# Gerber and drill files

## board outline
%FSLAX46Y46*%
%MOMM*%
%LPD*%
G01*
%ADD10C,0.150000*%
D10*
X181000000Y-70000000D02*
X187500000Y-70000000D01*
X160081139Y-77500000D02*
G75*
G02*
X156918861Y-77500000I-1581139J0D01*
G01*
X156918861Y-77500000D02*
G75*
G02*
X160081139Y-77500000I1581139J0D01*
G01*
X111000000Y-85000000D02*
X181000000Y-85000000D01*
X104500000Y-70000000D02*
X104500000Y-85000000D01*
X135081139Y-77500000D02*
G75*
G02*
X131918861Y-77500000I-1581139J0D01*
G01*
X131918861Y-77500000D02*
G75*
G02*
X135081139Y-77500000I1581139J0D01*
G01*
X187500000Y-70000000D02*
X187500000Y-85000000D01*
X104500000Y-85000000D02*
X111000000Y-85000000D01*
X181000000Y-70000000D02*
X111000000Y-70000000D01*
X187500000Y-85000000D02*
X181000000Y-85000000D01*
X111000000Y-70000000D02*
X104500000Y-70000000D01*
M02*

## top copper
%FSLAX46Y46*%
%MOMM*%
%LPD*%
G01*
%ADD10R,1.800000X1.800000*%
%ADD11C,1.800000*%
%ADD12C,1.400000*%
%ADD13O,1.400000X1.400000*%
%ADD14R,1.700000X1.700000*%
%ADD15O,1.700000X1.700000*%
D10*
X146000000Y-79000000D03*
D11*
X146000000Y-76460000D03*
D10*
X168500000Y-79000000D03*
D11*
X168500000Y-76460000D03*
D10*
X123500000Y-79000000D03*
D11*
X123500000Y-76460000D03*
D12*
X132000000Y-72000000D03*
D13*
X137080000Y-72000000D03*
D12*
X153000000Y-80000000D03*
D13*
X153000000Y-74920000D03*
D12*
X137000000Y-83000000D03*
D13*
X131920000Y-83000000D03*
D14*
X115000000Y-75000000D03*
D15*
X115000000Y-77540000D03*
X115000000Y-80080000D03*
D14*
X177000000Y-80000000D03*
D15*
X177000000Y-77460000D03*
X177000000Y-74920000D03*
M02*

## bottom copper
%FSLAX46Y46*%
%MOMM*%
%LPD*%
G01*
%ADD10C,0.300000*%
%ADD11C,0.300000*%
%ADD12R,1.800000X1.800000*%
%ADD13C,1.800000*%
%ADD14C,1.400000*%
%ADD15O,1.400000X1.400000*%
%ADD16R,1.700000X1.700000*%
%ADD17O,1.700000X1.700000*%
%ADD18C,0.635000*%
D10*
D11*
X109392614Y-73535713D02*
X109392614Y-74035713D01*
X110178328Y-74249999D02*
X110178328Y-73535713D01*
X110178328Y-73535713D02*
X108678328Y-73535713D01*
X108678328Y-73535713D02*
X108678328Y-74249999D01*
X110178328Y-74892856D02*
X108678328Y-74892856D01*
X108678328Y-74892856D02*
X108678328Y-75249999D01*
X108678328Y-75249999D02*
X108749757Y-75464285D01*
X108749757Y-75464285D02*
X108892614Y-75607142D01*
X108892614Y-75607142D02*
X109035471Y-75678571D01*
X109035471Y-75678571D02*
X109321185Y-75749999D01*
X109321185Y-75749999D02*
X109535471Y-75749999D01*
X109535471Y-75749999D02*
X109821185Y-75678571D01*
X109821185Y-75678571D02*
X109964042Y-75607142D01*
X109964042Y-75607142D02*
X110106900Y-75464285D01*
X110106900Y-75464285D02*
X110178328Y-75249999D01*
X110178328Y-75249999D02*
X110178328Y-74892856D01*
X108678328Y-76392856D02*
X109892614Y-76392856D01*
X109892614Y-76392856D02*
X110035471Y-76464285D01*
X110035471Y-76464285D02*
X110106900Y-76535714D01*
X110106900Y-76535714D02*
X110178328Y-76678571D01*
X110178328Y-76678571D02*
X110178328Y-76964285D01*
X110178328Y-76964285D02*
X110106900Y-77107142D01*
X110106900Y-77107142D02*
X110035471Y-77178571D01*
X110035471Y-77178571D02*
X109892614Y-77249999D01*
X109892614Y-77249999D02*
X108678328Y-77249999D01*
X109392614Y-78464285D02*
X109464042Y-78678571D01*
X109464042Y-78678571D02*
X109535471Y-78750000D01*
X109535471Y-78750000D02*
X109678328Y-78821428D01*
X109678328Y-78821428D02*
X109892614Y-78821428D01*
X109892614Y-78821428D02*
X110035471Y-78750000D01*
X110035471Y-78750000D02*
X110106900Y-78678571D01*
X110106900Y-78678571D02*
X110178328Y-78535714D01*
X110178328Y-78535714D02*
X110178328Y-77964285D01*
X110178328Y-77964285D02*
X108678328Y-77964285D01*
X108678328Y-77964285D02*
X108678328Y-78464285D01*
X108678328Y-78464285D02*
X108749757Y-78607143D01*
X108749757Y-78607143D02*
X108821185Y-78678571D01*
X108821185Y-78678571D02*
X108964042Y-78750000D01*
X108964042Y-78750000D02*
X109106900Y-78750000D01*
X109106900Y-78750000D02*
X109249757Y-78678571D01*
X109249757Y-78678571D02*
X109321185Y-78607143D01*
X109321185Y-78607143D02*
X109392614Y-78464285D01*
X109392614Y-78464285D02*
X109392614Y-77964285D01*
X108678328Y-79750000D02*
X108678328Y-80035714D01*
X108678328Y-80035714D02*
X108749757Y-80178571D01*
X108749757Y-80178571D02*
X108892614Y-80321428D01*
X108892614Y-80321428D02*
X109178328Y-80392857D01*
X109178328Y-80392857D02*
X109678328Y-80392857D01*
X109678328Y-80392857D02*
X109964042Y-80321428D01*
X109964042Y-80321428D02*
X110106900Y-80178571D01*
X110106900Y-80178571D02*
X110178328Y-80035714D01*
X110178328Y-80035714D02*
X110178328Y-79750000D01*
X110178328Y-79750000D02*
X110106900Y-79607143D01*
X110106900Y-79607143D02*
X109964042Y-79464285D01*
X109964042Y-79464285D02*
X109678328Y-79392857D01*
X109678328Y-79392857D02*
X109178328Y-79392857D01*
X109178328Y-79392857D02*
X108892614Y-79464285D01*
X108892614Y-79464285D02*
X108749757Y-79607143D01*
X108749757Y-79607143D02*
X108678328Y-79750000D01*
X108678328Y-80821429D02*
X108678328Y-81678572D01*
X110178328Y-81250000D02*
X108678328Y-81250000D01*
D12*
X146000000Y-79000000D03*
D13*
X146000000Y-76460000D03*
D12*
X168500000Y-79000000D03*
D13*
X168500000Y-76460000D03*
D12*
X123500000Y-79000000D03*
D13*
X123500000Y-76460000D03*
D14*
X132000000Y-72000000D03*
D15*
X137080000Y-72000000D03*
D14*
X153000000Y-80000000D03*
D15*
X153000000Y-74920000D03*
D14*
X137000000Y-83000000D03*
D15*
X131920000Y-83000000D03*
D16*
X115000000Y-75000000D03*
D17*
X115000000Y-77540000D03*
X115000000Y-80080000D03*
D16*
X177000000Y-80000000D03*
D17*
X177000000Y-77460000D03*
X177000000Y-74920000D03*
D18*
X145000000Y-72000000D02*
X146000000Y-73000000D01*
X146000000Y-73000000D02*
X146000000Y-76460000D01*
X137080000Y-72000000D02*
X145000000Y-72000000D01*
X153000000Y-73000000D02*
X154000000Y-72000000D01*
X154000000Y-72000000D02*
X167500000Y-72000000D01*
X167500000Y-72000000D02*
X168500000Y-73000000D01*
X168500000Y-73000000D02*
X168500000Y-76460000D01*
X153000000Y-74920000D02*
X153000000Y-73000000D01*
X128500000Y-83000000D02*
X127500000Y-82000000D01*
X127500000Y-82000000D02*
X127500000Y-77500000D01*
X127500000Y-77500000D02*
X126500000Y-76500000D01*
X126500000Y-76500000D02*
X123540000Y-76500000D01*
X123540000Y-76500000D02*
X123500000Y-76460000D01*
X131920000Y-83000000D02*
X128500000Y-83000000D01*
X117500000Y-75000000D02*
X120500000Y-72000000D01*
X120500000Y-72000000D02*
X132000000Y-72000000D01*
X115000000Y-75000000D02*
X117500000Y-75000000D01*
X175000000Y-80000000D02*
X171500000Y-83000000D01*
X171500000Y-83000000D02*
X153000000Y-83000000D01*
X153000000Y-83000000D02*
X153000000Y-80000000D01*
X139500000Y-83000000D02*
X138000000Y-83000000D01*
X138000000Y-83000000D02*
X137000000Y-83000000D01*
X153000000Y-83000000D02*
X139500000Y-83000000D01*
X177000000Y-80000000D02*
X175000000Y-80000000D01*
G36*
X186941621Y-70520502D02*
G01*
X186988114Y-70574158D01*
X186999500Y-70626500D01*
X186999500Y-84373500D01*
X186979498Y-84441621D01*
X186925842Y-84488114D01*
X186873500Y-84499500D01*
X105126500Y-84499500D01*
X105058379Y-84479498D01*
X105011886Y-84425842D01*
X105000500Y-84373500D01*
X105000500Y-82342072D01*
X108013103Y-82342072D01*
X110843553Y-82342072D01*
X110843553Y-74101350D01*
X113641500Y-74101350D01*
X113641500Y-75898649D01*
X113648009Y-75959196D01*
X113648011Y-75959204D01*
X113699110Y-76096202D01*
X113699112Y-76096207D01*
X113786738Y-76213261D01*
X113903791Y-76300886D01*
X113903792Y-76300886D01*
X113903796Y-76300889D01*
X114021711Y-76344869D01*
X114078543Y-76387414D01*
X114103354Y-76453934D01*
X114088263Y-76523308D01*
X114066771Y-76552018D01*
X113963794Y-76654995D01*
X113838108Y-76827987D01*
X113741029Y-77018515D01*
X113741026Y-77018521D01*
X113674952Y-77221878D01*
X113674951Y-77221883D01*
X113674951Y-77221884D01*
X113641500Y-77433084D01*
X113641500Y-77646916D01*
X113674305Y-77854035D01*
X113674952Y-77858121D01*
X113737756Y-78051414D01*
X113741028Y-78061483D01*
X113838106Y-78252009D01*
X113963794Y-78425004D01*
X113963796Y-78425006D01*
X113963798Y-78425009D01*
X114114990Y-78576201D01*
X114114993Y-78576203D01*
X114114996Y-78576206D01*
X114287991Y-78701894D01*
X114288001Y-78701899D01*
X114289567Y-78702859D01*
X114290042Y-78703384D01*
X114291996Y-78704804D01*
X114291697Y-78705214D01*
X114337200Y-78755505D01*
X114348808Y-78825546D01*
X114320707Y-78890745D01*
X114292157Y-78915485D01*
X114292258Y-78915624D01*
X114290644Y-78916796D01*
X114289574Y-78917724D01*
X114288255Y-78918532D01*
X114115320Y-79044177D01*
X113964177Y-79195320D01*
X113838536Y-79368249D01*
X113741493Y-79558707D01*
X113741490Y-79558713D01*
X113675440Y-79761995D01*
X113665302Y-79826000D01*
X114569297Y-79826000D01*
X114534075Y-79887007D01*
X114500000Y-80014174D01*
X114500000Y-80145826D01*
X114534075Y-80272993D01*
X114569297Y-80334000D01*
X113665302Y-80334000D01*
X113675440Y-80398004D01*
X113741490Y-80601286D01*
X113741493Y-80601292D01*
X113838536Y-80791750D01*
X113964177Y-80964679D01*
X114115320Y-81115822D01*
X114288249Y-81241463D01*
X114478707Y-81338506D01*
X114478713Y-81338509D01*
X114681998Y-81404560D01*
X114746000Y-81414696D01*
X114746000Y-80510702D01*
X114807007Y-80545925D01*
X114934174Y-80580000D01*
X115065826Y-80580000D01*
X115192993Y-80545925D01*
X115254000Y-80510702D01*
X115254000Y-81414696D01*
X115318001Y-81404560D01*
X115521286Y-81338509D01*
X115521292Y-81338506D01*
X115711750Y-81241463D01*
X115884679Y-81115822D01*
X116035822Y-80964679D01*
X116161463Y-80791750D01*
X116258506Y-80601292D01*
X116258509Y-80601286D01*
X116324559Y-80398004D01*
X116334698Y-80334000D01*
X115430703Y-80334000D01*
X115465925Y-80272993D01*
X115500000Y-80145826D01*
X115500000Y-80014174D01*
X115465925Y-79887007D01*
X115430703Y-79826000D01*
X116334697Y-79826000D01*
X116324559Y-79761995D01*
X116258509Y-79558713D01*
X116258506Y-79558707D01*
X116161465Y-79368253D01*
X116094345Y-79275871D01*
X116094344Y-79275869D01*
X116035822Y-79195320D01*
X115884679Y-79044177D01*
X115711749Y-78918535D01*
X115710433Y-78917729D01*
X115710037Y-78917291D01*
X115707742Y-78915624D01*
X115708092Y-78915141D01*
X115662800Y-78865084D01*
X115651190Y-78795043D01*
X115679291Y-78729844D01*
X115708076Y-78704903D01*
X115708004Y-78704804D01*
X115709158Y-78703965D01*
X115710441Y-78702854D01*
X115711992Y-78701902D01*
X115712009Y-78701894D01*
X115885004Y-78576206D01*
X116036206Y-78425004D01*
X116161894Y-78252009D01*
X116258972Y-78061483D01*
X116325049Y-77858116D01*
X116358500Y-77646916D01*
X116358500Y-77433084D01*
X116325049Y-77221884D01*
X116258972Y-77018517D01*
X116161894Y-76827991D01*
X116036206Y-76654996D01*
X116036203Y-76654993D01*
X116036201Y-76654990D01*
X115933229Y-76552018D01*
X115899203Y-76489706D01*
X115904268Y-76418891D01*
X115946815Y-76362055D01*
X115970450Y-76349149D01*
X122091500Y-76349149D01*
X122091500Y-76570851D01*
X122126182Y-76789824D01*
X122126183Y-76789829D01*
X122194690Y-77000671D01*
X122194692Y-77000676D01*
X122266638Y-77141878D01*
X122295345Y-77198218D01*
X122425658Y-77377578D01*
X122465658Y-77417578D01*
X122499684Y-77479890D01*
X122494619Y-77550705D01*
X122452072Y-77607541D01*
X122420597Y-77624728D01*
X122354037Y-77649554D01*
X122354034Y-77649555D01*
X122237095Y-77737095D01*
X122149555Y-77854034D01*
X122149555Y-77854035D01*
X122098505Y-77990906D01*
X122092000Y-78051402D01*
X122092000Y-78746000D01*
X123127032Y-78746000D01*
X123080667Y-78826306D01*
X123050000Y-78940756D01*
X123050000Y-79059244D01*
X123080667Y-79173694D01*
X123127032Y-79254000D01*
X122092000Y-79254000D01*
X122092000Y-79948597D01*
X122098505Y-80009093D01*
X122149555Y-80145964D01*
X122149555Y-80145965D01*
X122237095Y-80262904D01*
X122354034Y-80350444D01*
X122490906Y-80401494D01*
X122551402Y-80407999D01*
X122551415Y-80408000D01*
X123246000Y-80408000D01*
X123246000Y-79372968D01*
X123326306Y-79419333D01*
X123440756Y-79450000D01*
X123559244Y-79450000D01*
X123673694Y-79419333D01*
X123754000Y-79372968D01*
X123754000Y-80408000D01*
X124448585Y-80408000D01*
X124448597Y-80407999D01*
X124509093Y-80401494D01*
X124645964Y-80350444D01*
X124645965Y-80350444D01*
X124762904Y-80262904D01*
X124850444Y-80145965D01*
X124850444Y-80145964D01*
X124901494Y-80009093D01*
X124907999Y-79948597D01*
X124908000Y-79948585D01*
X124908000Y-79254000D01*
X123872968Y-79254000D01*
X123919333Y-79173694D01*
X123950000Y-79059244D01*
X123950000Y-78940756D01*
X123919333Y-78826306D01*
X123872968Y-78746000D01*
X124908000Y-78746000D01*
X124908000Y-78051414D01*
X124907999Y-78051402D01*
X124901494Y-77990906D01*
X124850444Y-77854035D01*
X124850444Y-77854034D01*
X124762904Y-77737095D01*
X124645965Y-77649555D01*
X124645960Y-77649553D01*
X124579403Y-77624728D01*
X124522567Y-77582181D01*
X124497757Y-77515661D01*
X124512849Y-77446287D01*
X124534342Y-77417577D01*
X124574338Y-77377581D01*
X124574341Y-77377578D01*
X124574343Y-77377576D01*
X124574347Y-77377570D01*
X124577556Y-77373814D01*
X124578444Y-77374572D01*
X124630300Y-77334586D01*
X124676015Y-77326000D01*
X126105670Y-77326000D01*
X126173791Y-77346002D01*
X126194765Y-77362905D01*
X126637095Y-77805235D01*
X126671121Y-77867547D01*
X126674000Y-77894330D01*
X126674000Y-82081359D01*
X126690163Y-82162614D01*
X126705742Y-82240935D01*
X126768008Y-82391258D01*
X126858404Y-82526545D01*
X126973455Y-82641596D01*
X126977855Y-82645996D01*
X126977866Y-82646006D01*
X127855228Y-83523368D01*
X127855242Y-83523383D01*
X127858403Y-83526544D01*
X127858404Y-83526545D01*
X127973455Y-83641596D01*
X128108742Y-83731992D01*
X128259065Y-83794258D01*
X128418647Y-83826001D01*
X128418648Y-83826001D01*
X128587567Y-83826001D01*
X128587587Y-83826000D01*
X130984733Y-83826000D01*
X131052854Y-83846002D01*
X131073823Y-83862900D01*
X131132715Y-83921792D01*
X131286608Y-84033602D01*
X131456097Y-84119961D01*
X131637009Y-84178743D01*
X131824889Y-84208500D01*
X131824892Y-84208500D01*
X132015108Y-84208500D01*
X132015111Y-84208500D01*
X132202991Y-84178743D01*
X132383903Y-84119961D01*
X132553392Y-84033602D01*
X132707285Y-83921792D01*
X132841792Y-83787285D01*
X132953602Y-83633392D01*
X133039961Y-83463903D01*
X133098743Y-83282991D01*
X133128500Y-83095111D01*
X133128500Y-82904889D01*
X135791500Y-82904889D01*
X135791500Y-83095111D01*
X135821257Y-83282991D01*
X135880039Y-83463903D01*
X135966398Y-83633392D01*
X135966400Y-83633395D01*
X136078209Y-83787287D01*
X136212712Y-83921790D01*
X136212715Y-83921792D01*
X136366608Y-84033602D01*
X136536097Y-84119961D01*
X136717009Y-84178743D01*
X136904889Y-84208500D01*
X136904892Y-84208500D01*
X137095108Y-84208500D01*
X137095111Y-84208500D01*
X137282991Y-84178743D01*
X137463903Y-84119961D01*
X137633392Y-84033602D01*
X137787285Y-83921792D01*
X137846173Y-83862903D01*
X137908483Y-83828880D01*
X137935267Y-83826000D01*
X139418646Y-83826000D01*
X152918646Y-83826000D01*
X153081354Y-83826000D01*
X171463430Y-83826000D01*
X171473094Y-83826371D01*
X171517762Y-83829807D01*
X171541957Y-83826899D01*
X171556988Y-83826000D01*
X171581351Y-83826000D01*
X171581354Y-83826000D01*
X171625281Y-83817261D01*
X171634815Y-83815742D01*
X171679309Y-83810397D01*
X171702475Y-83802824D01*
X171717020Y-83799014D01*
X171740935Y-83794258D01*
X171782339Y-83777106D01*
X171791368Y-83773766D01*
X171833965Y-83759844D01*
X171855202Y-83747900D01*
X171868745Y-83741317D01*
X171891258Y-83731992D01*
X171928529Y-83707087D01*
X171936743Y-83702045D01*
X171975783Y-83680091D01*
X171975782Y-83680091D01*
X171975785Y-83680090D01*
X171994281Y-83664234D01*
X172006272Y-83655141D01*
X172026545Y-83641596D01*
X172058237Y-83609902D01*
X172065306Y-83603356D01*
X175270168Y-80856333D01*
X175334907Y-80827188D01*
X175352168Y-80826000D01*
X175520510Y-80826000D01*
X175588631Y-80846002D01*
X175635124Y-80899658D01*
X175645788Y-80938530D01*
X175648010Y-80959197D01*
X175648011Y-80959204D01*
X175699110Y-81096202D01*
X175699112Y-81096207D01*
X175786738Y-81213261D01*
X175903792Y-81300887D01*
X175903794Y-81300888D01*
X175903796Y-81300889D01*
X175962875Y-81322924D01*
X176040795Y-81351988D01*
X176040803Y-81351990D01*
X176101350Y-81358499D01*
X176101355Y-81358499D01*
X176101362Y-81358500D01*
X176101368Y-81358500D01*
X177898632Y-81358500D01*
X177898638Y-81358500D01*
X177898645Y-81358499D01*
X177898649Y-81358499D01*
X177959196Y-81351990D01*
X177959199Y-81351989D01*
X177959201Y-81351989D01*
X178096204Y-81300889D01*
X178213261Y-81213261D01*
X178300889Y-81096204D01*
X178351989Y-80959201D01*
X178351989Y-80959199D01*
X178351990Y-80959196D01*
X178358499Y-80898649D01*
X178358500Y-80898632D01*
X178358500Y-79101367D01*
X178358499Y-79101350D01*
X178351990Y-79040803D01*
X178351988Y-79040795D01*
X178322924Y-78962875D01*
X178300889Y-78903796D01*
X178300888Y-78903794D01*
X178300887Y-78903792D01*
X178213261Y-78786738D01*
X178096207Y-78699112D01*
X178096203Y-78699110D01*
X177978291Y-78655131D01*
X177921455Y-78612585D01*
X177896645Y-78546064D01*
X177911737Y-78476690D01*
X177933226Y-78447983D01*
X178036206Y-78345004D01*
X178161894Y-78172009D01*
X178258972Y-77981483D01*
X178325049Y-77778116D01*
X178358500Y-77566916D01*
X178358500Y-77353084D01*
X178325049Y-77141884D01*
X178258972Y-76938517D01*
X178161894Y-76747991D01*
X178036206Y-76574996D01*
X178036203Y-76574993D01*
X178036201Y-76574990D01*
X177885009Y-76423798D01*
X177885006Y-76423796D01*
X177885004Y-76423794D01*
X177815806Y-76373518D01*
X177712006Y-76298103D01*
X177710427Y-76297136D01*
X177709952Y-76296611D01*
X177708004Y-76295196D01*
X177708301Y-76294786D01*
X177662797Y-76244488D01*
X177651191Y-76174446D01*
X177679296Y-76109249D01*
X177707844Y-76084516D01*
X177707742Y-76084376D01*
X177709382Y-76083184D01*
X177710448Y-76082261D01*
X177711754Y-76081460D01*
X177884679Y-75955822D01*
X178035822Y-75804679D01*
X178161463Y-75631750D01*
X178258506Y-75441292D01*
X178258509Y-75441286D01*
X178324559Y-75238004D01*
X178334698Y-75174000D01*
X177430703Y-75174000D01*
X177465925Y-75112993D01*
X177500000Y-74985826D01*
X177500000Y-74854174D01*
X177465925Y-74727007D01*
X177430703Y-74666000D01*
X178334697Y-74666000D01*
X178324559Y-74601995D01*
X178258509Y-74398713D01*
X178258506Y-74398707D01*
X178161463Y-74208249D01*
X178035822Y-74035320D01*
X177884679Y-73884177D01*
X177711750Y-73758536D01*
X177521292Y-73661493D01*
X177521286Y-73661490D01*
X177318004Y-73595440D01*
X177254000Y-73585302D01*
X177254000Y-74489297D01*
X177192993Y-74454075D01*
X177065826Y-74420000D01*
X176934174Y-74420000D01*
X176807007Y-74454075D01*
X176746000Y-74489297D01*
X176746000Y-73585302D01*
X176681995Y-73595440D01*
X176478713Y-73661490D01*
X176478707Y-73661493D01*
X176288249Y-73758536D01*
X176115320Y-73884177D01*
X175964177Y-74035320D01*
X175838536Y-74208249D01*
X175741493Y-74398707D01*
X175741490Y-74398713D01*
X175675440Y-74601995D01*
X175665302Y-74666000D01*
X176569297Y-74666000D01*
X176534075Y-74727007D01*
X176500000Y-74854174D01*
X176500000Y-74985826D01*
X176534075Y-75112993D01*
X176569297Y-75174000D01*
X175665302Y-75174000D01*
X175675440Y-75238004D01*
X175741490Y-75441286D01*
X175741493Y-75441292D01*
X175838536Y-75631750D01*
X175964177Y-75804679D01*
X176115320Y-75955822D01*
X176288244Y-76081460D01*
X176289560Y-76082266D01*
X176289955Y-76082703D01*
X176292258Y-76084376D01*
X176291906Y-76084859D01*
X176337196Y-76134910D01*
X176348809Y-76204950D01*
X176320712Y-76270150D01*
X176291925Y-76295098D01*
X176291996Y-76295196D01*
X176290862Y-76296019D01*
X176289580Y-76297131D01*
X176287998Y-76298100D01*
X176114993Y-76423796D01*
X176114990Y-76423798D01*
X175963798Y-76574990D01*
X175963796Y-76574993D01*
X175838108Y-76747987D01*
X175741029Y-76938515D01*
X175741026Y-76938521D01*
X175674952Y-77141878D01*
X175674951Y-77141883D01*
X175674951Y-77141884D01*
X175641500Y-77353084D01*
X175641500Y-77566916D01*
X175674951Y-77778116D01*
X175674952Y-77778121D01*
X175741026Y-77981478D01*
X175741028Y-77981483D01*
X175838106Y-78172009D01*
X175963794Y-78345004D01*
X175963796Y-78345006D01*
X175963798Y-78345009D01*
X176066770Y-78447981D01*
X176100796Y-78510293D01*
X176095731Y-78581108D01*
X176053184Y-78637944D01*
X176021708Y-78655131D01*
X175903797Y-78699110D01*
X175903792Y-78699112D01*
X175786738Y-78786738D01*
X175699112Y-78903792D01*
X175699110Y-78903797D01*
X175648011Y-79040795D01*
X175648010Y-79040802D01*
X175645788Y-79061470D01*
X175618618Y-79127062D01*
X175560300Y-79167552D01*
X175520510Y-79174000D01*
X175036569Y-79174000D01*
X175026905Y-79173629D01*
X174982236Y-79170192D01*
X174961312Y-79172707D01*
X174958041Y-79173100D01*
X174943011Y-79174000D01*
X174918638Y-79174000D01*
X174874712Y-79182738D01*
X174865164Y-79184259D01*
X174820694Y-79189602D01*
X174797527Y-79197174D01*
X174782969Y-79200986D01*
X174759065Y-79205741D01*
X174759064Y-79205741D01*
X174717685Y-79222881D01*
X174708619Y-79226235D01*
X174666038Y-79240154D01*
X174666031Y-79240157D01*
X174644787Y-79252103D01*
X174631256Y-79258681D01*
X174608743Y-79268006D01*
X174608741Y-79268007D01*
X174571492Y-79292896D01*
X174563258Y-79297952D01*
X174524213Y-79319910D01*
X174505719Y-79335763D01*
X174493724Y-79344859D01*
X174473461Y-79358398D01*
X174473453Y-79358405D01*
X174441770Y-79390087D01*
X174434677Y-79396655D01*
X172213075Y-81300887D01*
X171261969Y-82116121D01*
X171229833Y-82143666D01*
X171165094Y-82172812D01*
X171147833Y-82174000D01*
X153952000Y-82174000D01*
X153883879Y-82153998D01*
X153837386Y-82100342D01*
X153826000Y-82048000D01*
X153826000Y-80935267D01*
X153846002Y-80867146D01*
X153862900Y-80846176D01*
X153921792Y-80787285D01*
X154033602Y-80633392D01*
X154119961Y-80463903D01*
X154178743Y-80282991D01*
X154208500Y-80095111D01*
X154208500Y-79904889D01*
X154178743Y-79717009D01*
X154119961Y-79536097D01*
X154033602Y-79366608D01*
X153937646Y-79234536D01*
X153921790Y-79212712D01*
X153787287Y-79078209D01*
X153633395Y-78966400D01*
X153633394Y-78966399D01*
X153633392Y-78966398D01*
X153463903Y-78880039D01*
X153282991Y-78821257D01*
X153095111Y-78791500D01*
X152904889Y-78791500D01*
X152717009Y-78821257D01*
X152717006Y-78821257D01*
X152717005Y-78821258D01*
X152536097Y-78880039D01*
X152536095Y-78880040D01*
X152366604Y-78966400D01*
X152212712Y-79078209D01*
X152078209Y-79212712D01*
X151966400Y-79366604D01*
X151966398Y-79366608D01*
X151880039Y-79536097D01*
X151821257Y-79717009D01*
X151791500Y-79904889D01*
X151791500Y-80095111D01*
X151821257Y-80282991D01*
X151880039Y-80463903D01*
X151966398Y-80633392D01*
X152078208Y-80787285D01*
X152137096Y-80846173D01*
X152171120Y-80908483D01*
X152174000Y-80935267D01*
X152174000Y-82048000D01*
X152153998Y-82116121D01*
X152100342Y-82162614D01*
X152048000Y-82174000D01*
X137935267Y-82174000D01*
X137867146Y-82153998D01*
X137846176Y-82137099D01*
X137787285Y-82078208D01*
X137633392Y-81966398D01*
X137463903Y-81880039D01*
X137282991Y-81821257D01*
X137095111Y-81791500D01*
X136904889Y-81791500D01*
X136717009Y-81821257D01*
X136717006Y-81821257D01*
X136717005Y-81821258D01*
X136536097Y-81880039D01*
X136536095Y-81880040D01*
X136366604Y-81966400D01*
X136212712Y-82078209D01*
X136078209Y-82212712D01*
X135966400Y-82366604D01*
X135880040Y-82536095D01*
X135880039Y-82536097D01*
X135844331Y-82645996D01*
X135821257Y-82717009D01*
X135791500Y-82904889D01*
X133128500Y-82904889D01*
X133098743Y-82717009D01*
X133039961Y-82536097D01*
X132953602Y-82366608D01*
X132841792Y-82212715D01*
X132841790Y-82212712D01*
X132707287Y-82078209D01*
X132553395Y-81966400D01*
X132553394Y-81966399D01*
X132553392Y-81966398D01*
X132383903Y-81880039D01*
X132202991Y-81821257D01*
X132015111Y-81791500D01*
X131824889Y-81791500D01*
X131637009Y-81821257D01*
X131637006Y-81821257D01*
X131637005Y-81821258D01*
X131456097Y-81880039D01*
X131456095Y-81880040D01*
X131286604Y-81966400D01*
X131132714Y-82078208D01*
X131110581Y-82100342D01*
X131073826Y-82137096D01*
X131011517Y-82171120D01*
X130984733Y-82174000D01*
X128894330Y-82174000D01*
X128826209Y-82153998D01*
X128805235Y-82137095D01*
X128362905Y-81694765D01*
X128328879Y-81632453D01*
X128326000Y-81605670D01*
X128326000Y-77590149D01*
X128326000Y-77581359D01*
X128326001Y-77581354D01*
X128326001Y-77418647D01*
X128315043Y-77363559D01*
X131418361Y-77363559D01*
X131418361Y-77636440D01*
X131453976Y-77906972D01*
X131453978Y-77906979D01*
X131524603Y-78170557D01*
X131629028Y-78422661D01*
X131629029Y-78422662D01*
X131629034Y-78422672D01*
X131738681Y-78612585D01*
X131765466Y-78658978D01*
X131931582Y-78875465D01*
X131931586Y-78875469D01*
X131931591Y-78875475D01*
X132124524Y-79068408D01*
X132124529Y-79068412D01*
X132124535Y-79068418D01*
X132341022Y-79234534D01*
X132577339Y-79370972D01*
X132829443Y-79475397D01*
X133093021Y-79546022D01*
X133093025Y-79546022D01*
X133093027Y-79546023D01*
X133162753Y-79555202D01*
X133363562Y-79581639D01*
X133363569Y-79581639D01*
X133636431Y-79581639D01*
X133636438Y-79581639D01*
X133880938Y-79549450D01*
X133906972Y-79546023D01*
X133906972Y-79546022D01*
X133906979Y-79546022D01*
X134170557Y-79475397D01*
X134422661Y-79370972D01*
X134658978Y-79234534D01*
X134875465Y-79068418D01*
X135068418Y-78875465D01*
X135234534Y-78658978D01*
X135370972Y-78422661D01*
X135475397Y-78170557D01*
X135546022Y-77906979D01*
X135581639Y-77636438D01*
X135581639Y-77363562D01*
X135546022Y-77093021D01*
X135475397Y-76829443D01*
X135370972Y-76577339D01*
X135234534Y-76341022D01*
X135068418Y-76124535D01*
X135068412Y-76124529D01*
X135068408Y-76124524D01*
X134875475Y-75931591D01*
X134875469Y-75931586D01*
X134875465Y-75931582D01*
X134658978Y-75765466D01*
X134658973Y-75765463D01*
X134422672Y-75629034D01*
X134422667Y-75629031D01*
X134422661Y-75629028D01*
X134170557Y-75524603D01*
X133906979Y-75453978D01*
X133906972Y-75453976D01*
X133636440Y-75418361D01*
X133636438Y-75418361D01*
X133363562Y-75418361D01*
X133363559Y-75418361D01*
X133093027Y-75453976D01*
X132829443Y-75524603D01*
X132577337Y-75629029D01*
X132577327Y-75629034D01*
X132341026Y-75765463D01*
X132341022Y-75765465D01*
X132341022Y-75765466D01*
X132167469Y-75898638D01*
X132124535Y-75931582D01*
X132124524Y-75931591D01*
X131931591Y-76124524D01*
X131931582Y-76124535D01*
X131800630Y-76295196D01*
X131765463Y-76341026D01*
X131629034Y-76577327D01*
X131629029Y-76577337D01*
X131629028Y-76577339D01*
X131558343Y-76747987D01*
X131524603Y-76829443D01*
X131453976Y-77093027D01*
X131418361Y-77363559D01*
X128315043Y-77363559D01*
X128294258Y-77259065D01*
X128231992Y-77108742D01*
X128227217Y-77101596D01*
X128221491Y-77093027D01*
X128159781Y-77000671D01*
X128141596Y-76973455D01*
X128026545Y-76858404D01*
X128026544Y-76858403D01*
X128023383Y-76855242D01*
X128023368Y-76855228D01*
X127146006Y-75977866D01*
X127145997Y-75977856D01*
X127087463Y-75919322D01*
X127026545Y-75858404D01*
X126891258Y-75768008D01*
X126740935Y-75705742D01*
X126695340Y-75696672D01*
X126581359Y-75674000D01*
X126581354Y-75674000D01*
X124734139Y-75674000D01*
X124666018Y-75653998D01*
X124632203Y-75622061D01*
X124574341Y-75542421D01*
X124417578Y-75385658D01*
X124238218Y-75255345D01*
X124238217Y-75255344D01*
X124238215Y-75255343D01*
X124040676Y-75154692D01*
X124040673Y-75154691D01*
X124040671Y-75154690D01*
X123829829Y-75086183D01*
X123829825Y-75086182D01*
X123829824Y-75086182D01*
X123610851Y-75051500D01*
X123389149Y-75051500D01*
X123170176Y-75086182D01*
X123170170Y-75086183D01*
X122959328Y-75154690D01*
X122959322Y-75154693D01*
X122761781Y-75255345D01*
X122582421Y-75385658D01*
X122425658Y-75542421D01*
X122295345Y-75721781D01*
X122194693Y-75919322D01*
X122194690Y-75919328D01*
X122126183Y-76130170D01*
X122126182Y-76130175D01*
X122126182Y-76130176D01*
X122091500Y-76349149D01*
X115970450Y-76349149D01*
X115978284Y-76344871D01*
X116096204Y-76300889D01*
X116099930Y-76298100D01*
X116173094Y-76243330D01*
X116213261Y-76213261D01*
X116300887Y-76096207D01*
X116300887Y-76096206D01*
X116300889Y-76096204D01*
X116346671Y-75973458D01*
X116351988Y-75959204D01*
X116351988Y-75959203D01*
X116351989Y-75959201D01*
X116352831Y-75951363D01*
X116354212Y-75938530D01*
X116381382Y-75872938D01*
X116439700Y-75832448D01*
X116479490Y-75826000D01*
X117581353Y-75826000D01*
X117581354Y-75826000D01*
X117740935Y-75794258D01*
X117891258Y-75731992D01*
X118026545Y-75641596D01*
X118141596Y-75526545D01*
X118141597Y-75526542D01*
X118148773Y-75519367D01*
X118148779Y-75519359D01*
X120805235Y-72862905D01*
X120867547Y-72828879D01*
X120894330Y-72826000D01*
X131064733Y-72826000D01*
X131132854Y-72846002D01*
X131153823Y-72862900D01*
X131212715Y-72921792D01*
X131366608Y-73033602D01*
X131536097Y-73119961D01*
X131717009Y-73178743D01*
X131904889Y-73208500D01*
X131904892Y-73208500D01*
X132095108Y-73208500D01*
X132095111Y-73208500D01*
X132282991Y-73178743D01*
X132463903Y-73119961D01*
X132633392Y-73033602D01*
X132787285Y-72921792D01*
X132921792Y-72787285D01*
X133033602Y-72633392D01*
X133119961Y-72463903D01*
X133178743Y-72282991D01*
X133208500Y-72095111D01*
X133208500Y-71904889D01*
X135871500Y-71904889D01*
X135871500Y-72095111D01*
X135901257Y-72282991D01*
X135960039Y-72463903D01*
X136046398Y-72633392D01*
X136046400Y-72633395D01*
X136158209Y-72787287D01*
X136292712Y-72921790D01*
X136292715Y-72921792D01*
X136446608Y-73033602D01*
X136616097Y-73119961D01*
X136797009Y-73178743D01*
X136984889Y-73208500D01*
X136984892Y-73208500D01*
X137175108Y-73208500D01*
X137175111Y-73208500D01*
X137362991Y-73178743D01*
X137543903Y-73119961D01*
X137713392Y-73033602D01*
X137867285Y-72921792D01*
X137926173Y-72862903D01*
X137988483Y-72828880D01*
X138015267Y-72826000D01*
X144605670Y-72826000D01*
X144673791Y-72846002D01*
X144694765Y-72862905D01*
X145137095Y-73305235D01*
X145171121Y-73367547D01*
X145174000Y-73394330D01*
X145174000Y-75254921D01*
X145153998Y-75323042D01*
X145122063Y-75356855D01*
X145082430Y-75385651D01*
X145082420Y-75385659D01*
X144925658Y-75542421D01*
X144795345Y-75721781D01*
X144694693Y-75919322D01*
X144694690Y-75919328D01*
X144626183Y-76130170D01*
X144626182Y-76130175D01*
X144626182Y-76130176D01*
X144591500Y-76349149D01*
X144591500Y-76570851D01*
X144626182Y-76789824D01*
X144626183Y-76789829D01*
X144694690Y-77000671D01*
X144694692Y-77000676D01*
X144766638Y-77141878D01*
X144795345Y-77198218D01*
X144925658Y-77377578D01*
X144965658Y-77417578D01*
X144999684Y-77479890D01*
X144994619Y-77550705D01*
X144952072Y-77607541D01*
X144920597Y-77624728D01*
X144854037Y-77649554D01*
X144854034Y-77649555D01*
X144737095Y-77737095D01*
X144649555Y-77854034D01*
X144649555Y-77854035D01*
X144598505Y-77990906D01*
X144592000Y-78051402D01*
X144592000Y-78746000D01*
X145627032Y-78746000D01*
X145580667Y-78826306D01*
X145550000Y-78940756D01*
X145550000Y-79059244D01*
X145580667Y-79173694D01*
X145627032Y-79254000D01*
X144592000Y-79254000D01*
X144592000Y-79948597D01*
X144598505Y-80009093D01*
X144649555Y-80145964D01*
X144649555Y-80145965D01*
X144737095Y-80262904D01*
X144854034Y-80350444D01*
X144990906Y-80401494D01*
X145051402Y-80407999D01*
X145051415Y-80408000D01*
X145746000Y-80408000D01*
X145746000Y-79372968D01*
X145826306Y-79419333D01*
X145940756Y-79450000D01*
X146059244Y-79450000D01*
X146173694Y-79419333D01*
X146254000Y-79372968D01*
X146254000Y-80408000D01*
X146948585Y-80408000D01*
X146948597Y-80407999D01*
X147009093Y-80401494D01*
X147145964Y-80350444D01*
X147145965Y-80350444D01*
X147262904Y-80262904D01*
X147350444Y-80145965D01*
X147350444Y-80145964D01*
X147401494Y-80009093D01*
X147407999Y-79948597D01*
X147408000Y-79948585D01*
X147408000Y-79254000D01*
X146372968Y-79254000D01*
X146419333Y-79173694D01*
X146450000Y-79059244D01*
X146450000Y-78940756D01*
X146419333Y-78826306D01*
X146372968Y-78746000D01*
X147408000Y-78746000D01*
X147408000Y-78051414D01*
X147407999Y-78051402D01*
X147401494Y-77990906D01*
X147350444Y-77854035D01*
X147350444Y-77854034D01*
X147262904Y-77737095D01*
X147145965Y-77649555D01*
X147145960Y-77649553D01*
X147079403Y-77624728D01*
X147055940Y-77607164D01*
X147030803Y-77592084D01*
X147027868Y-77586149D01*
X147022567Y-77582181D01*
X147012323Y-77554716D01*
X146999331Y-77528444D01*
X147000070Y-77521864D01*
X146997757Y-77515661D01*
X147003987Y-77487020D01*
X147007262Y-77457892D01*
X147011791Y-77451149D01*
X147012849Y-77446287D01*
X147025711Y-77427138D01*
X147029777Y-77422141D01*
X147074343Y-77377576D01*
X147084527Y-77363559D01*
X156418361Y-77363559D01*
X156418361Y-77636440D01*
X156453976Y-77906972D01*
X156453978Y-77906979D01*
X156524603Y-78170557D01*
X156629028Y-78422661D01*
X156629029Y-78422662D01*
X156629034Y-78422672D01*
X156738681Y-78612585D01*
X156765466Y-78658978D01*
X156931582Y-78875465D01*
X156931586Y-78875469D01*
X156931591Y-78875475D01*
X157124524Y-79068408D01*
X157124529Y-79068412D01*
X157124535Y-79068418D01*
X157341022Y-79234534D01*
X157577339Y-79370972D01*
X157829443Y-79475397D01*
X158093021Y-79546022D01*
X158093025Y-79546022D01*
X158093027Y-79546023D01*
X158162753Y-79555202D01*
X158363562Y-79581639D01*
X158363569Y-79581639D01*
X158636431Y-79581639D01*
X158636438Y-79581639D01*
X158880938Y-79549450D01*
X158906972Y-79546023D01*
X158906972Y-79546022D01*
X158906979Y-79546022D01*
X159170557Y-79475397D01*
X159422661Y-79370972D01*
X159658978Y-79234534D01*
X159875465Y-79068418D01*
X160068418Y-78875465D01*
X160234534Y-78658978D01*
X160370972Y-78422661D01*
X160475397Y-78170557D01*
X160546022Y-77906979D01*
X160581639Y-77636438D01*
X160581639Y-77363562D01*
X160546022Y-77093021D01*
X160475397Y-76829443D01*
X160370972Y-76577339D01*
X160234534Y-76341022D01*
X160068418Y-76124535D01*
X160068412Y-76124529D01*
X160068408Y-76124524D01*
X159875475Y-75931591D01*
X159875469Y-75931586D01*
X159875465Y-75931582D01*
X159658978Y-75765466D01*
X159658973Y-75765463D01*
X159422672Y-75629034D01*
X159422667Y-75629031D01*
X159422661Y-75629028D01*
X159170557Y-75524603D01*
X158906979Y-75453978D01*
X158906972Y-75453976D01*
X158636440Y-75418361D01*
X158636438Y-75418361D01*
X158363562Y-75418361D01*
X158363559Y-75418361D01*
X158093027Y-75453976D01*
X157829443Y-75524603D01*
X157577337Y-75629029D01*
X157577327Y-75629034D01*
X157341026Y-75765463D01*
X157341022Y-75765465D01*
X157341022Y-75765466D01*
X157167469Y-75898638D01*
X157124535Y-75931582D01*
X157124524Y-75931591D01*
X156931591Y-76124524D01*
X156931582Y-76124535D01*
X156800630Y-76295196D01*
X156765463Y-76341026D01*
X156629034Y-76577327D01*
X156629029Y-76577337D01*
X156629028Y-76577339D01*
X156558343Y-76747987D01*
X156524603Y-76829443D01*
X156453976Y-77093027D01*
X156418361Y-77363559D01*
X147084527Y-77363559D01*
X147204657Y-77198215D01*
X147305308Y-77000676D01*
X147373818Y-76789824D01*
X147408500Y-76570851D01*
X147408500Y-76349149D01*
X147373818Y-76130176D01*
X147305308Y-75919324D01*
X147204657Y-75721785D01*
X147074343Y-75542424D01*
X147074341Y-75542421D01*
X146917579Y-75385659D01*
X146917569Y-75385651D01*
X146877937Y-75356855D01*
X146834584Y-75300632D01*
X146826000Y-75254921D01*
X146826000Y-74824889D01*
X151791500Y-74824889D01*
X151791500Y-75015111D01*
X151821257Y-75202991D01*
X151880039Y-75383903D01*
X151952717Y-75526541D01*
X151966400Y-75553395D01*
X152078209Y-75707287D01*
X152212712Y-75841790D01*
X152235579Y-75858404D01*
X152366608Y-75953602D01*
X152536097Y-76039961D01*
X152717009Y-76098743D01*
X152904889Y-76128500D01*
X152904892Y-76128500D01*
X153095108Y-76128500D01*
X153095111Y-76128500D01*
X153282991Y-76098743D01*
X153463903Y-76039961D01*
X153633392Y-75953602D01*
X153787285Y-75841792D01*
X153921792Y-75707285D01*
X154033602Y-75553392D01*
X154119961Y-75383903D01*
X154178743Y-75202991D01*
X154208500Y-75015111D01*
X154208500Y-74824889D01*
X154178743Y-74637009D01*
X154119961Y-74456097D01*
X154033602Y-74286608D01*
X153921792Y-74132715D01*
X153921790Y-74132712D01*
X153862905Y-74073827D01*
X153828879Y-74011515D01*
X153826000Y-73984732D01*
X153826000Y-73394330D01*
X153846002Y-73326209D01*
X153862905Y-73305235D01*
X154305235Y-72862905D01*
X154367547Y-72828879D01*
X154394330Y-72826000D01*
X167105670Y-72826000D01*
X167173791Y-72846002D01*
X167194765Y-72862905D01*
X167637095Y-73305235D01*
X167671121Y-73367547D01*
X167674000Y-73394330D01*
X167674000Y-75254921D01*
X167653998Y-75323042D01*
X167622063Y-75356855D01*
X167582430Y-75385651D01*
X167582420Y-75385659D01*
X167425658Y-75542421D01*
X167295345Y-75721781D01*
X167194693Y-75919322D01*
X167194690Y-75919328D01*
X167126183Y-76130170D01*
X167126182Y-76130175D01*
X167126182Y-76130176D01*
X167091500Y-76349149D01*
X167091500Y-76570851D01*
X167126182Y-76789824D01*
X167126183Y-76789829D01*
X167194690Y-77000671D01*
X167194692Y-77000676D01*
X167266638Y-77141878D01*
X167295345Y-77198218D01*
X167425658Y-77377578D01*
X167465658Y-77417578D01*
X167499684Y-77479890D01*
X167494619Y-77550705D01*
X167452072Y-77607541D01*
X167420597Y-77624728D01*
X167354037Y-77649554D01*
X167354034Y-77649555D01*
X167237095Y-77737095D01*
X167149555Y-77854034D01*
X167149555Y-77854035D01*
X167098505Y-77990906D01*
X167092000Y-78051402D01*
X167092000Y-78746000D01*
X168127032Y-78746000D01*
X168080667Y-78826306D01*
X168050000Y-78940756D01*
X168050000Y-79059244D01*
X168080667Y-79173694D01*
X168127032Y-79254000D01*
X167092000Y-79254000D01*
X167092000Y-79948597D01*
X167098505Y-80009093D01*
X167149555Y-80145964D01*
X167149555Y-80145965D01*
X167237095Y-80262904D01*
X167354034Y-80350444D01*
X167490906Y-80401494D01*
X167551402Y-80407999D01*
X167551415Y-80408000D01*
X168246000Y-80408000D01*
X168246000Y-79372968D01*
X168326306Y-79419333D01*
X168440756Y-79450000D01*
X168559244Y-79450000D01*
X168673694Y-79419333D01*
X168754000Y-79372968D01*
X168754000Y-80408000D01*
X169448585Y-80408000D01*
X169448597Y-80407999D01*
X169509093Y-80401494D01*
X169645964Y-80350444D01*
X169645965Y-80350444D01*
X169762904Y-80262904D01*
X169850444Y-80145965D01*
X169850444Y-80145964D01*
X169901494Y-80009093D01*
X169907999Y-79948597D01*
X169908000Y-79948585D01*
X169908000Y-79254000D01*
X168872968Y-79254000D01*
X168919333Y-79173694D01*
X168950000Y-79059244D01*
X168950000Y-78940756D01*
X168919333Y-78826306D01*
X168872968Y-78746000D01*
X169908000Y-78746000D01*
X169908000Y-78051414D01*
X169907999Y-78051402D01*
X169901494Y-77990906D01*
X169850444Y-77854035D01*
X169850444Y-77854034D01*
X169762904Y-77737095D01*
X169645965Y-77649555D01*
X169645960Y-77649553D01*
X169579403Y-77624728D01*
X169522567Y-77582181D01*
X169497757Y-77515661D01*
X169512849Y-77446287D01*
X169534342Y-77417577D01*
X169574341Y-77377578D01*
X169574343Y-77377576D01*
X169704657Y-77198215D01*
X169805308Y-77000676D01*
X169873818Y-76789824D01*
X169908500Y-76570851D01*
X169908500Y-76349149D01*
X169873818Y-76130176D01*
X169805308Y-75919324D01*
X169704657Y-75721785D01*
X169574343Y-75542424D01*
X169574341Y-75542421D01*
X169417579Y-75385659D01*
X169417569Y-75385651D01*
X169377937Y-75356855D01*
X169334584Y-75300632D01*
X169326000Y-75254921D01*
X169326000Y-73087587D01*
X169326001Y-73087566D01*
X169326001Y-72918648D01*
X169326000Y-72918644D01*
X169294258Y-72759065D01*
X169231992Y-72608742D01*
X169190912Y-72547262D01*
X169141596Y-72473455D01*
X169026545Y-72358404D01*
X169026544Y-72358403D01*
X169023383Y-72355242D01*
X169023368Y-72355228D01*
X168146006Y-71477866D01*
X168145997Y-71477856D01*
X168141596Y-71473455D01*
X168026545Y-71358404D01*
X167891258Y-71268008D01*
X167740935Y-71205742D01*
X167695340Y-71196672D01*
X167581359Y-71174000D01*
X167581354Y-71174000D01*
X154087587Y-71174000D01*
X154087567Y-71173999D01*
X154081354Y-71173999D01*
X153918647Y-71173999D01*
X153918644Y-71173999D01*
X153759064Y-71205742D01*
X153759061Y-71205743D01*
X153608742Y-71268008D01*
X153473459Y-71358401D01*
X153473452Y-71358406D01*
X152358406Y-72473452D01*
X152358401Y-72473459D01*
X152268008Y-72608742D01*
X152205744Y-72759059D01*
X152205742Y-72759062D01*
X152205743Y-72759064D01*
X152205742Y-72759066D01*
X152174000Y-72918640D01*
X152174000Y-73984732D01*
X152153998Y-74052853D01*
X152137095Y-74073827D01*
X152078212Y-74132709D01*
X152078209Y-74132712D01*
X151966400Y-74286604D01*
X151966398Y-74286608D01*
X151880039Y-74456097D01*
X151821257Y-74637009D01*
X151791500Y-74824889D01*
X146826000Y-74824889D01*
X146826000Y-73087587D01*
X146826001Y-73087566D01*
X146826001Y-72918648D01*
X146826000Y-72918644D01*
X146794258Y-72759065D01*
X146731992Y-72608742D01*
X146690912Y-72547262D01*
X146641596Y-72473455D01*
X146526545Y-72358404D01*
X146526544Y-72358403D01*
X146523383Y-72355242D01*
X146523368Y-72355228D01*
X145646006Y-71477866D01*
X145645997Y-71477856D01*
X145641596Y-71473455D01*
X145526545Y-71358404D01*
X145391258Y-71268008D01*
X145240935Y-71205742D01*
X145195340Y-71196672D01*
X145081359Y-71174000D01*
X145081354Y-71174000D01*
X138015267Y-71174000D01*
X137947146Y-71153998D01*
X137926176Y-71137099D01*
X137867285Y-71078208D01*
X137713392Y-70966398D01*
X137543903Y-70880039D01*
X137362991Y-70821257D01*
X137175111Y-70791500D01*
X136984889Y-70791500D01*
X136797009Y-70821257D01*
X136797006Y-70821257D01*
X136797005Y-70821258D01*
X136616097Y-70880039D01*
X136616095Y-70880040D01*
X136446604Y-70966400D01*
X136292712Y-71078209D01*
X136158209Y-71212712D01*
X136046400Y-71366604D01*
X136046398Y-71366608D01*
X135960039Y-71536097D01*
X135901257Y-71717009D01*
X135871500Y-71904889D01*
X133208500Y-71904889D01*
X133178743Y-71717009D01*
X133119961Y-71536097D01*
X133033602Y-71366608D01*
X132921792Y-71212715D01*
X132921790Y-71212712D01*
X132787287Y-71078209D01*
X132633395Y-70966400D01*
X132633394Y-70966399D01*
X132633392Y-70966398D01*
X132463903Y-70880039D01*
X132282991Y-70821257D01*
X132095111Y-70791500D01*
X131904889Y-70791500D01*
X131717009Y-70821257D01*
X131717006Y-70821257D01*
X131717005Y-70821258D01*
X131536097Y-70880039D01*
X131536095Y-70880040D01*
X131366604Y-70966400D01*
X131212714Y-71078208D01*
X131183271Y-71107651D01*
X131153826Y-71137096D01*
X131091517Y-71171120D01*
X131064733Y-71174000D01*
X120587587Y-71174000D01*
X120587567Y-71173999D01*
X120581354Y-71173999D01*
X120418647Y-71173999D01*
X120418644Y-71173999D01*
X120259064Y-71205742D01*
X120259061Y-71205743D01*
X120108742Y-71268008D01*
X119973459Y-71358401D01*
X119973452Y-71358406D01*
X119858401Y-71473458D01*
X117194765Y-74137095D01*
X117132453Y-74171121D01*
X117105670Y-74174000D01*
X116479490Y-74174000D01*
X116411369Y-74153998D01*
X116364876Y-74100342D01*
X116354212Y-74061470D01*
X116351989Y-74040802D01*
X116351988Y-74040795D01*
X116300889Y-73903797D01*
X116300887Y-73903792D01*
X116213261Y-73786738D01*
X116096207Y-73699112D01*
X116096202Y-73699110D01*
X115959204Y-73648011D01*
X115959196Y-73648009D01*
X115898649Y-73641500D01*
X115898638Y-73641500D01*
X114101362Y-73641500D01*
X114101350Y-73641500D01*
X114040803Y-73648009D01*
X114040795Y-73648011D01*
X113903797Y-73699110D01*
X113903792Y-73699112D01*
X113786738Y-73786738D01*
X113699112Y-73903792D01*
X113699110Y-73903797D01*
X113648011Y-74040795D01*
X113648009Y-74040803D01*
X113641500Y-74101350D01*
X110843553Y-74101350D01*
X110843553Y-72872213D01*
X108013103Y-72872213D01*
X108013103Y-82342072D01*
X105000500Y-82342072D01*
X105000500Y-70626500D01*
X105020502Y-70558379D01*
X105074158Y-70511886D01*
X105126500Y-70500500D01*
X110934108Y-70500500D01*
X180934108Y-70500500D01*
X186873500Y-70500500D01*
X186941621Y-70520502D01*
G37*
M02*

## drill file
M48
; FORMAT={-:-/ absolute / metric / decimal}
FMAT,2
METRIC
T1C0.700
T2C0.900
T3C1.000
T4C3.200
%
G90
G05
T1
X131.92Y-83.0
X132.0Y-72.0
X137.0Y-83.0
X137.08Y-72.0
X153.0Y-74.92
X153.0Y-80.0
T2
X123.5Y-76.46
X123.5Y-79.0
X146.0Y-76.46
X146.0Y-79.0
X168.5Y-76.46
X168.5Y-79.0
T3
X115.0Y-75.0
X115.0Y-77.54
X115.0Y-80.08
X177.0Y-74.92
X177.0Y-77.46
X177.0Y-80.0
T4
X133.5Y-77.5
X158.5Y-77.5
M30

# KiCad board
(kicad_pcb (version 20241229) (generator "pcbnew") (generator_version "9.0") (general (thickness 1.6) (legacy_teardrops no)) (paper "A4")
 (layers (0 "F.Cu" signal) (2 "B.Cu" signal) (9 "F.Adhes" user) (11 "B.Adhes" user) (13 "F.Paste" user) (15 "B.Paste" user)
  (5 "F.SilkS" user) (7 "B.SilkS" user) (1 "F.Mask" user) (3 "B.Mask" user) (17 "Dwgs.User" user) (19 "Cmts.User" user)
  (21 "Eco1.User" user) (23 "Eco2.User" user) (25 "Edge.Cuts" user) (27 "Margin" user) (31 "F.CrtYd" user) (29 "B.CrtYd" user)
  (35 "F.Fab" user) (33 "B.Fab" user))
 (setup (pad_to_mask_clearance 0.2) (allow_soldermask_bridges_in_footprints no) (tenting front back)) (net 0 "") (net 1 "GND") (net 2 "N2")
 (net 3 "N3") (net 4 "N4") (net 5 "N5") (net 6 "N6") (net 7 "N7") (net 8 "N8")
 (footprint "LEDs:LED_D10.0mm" (layer "F.Cu") (at 146 79 90)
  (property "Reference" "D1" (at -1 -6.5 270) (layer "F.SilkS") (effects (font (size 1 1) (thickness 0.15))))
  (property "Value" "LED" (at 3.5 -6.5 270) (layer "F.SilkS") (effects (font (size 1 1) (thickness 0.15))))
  (pad "1" thru_hole rect (at 0 0 90) (size 1.8 1.8) (drill 0.9) (layers "*.Cu" "*.Mask") (remove_unused_layers no) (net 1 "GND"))
  (pad "2" thru_hole circle (at 2.54 0 90) (size 1.8 1.8) (drill 0.9) (layers "*.Cu" "*.Mask") (remove_unused_layers no) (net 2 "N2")))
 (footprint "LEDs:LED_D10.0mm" (layer "F.Cu") (at 168.5 79 90)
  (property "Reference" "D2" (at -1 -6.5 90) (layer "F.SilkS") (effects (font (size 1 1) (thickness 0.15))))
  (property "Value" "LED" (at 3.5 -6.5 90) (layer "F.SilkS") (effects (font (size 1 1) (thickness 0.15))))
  (pad "1" thru_hole rect (at 0 0 90) (size 1.8 1.8) (drill 0.9) (layers "*.Cu" "*.Mask") (remove_unused_layers no) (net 1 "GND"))
  (pad "2" thru_hole circle (at 2.54 0 90) (size 1.8 1.8) (drill 0.9) (layers "*.Cu" "*.Mask") (remove_unused_layers no) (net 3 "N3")))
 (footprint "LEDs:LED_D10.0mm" (layer "F.Cu") (at 123.5 79 90)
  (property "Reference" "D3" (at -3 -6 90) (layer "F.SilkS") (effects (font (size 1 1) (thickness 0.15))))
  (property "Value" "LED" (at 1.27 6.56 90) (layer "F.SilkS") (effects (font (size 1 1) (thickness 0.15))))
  (pad "1" thru_hole rect (at 0 0 90) (size 1.8 1.8) (drill 0.9) (layers "*.Cu" "*.Mask") (remove_unused_layers no) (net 1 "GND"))
  (pad "2" thru_hole circle (at 2.54 0 90) (size 1.8 1.8) (drill 0.9) (layers "*.Cu" "*.Mask") (remove_unused_layers no) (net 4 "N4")))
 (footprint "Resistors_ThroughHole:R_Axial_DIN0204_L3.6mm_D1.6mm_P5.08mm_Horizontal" (layer "F.Cu") (at 132 72)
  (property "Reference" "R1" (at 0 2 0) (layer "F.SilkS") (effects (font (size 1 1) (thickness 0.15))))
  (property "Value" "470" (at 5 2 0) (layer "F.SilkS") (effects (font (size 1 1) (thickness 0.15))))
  (pad "1" thru_hole circle (at 0 0) (size 1.4 1.4) (drill 0.7) (layers "*.Cu" "*.Mask") (remove_unused_layers no) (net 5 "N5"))
  (pad "2" thru_hole oval (at 5.08 0) (size 1.4 1.4) (drill 0.7) (layers "*.Cu" "*.Mask") (remove_unused_layers no) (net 2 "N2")))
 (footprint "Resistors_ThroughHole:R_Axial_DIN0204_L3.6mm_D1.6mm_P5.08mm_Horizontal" (layer "F.Cu") (at 153 80 90)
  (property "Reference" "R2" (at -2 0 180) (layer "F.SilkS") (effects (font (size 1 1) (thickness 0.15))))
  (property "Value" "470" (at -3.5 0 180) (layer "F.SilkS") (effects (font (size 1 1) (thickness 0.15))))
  (pad "1" thru_hole circle (at 0 0 90) (size 1.4 1.4) (drill 0.7) (layers "*.Cu" "*.Mask") (remove_unused_layers no) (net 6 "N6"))
  (pad "2" thru_hole oval (at 5.08 0 90) (size 1.4 1.4) (drill 0.7) (layers "*.Cu" "*.Mask") (remove_unused_layers no) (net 3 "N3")))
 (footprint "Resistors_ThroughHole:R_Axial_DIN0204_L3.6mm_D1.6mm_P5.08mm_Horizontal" (layer "F.Cu") (at 137 83 180)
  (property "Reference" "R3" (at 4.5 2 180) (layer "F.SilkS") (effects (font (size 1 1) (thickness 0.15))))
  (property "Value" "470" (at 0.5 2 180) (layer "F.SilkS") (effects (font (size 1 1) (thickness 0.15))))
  (pad "1" thru_hole circle (at 0 0 180) (size 1.4 1.4) (drill 0.7) (layers "*.Cu" "*.Mask") (remove_unused_layers no) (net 6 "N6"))
  (pad "2" thru_hole oval (at 5.08 0 180) (size 1.4 1.4) (drill 0.7) (layers "*.Cu" "*.Mask") (remove_unused_layers no) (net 4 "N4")))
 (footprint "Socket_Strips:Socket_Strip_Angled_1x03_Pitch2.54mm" (layer "F.Cu") (at 115 75)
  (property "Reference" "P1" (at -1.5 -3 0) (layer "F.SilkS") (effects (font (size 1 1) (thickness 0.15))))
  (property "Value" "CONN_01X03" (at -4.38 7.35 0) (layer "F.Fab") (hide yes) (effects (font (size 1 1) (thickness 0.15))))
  (pad "1" thru_hole rect (at 0 0) (size 1.7 1.7) (drill 1) (layers "*.Cu" "*.Mask") (remove_unused_layers no) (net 5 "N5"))
  (pad "2" thru_hole oval (at 0 2.54) (size 1.7 1.7) (drill 1) (layers "*.Cu" "*.Mask") (remove_unused_layers no) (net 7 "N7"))
  (pad "3" thru_hole oval (at 0 5.08) (size 1.7 1.7) (drill 1) (layers "*.Cu" "*.Mask") (remove_unused_layers no) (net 1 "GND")))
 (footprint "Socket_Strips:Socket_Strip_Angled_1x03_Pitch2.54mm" (layer "F.Cu") (at 177 80 180)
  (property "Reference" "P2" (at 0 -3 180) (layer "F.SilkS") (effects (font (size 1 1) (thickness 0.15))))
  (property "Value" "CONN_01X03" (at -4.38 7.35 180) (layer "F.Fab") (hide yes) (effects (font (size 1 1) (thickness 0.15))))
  (pad "1" thru_hole rect (at 0 0 180) (size 1.7 1.7) (drill 1) (layers "*.Cu" "*.Mask") (remove_unused_layers no) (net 6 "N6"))
  (pad "2" thru_hole oval (at 0 2.54 180) (size 1.7 1.7) (drill 1) (layers "*.Cu" "*.Mask") (remove_unused_layers no) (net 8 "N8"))
  (pad "3" thru_hole oval (at 0 5.08 180) (size 1.7 1.7) (drill 1) (layers "*.Cu" "*.Mask") (remove_unused_layers no) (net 1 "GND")))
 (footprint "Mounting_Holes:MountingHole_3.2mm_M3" (layer "F.Cu") (at 133.5 77.5)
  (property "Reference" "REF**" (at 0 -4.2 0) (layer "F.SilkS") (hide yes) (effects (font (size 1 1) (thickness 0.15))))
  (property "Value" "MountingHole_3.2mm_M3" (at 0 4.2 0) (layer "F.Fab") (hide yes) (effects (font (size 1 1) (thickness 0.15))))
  (pad "" np_thru_hole circle (at 0 0) (size 3.2 3.2) (drill 3.2) (layers "*.Cu" "*.Mask")))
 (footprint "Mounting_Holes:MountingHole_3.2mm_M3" (layer "F.Cu") (at 158.5 77.5)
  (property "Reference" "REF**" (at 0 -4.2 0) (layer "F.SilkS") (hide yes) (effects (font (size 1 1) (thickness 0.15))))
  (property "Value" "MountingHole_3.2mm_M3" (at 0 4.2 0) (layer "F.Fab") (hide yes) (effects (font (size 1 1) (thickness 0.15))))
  (pad "" np_thru_hole circle (at 0 0) (size 3.2 3.2) (drill 3.2) (layers "*.Cu" "*.Mask")))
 (gr_line (start 181 70) (end 187.5 70) (stroke (width 0.15) (type solid)) (layer "Edge.Cuts"))
 (gr_circle (center 158.5 77.5) (end 158 76) (stroke (width 0.15) (type solid)) (fill no) (layer "Edge.Cuts"))
 (gr_line (start 111 85) (end 181 85) (stroke (width 0.15) (type solid)) (layer "Edge.Cuts"))
 (gr_line (start 104.5 70) (end 104.5 85) (stroke (width 0.15) (type solid)) (layer "Edge.Cuts"))
 (gr_circle (center 133.5 77.5) (end 133 76) (stroke (width 0.15) (type solid)) (fill no) (layer "Edge.Cuts"))
 (gr_line (start 187.5 70) (end 187.5 85) (stroke (width 0.15) (type solid)) (layer "Edge.Cuts"))
 (gr_line (start 104.5 85) (end 111 85) (stroke (width 0.15) (type solid)) (layer "Edge.Cuts"))
 (gr_line (start 181 70) (end 111 70) (stroke (width 0.15) (type solid)) (layer "Edge.Cuts"))
 (gr_line (start 187.5 85) (end 181 85) (stroke (width 0.15) (type solid)) (layer "Edge.Cuts"))
 (gr_line (start 111 70) (end 104.5 70) (stroke (width 0.15) (type solid)) (layer "Edge.Cuts"))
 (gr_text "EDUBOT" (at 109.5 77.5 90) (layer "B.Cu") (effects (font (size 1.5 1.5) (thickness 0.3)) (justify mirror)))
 (segment (start 145 72) (end 146 73) (width 0.635) (layer "B.Cu") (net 2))
 (segment (start 146 73) (end 146 76.46) (width 0.635) (layer "B.Cu") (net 2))
 (segment (start 137.08 72) (end 145 72) (width 0.635) (layer "B.Cu") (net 2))
 (segment (start 153 73) (end 154 72) (width 0.635) (layer "B.Cu") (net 3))
 (segment (start 154 72) (end 167.5 72) (width 0.635) (layer "B.Cu") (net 3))
 (segment (start 167.5 72) (end 168.5 73) (width 0.635) (layer "B.Cu") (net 3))
 (segment (start 168.5 73) (end 168.5 76.46) (width 0.635) (layer "B.Cu") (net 3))
 (segment (start 153 74.92) (end 153 73) (width 0.635) (layer "B.Cu") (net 3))
 (segment (start 128.5 83) (end 127.5 82) (width 0.635) (layer "B.Cu") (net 4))
 (segment (start 127.5 82) (end 127.5 77.5) (width 0.635) (layer "B.Cu") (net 4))
 (segment (start 127.5 77.5) (end 126.5 76.5) (width 0.635) (layer "B.Cu") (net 4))
 (segment (start 126.5 76.5) (end 123.54 76.5) (width 0.635) (layer "B.Cu") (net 4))
 (segment (start 123.54 76.5) (end 123.5 76.46) (width 0.635) (layer "B.Cu") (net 4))
 (segment (start 131.92 83) (end 128.5 83) (width 0.635) (layer "B.Cu") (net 4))
 (segment (start 117.5 75) (end 120.5 72) (width 0.635) (layer "B.Cu") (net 5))
 (segment (start 120.5 72) (end 132 72) (width 0.635) (layer "B.Cu") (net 5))
 (segment (start 115 75) (end 117.5 75) (width 0.635) (layer "B.Cu") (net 5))
 (segment (start 175 80) (end 171.5 83) (width 0.635) (layer "B.Cu") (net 6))
 (segment (start 171.5 83) (end 153 83) (width 0.635) (layer "B.Cu") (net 6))
 (segment (start 153 83) (end 153 80) (width 0.635) (layer "B.Cu") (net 6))
 (segment (start 139.5 83) (end 138 83) (width 0.635) (layer "B.Cu") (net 6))
 (segment (start 138 83) (end 137 83) (width 0.635) (layer "B.Cu") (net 6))
 (segment (start 153 83) (end 139.5 83) (width 0.635) (layer "B.Cu") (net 6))
 (segment (start 177 80) (end 175 80) (width 0.635) (layer "B.Cu") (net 6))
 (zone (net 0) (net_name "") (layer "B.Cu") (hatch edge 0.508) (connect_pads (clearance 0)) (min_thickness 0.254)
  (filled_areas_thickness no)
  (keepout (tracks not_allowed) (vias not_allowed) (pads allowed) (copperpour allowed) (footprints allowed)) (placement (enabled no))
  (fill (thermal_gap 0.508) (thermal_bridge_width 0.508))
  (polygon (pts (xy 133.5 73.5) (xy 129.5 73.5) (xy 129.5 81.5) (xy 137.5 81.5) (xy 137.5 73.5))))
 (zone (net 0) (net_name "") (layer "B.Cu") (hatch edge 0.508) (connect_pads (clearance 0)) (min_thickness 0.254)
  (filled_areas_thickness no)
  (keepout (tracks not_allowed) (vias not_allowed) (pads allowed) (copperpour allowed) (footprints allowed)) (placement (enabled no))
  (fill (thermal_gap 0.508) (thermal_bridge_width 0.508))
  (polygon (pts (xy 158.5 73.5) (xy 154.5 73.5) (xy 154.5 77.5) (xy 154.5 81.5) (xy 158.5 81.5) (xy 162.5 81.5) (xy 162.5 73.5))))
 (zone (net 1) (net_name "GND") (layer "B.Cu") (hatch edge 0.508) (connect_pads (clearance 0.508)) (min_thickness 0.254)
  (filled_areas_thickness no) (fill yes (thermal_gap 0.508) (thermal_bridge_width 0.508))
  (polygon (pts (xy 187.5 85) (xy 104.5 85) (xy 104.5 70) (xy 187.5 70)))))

